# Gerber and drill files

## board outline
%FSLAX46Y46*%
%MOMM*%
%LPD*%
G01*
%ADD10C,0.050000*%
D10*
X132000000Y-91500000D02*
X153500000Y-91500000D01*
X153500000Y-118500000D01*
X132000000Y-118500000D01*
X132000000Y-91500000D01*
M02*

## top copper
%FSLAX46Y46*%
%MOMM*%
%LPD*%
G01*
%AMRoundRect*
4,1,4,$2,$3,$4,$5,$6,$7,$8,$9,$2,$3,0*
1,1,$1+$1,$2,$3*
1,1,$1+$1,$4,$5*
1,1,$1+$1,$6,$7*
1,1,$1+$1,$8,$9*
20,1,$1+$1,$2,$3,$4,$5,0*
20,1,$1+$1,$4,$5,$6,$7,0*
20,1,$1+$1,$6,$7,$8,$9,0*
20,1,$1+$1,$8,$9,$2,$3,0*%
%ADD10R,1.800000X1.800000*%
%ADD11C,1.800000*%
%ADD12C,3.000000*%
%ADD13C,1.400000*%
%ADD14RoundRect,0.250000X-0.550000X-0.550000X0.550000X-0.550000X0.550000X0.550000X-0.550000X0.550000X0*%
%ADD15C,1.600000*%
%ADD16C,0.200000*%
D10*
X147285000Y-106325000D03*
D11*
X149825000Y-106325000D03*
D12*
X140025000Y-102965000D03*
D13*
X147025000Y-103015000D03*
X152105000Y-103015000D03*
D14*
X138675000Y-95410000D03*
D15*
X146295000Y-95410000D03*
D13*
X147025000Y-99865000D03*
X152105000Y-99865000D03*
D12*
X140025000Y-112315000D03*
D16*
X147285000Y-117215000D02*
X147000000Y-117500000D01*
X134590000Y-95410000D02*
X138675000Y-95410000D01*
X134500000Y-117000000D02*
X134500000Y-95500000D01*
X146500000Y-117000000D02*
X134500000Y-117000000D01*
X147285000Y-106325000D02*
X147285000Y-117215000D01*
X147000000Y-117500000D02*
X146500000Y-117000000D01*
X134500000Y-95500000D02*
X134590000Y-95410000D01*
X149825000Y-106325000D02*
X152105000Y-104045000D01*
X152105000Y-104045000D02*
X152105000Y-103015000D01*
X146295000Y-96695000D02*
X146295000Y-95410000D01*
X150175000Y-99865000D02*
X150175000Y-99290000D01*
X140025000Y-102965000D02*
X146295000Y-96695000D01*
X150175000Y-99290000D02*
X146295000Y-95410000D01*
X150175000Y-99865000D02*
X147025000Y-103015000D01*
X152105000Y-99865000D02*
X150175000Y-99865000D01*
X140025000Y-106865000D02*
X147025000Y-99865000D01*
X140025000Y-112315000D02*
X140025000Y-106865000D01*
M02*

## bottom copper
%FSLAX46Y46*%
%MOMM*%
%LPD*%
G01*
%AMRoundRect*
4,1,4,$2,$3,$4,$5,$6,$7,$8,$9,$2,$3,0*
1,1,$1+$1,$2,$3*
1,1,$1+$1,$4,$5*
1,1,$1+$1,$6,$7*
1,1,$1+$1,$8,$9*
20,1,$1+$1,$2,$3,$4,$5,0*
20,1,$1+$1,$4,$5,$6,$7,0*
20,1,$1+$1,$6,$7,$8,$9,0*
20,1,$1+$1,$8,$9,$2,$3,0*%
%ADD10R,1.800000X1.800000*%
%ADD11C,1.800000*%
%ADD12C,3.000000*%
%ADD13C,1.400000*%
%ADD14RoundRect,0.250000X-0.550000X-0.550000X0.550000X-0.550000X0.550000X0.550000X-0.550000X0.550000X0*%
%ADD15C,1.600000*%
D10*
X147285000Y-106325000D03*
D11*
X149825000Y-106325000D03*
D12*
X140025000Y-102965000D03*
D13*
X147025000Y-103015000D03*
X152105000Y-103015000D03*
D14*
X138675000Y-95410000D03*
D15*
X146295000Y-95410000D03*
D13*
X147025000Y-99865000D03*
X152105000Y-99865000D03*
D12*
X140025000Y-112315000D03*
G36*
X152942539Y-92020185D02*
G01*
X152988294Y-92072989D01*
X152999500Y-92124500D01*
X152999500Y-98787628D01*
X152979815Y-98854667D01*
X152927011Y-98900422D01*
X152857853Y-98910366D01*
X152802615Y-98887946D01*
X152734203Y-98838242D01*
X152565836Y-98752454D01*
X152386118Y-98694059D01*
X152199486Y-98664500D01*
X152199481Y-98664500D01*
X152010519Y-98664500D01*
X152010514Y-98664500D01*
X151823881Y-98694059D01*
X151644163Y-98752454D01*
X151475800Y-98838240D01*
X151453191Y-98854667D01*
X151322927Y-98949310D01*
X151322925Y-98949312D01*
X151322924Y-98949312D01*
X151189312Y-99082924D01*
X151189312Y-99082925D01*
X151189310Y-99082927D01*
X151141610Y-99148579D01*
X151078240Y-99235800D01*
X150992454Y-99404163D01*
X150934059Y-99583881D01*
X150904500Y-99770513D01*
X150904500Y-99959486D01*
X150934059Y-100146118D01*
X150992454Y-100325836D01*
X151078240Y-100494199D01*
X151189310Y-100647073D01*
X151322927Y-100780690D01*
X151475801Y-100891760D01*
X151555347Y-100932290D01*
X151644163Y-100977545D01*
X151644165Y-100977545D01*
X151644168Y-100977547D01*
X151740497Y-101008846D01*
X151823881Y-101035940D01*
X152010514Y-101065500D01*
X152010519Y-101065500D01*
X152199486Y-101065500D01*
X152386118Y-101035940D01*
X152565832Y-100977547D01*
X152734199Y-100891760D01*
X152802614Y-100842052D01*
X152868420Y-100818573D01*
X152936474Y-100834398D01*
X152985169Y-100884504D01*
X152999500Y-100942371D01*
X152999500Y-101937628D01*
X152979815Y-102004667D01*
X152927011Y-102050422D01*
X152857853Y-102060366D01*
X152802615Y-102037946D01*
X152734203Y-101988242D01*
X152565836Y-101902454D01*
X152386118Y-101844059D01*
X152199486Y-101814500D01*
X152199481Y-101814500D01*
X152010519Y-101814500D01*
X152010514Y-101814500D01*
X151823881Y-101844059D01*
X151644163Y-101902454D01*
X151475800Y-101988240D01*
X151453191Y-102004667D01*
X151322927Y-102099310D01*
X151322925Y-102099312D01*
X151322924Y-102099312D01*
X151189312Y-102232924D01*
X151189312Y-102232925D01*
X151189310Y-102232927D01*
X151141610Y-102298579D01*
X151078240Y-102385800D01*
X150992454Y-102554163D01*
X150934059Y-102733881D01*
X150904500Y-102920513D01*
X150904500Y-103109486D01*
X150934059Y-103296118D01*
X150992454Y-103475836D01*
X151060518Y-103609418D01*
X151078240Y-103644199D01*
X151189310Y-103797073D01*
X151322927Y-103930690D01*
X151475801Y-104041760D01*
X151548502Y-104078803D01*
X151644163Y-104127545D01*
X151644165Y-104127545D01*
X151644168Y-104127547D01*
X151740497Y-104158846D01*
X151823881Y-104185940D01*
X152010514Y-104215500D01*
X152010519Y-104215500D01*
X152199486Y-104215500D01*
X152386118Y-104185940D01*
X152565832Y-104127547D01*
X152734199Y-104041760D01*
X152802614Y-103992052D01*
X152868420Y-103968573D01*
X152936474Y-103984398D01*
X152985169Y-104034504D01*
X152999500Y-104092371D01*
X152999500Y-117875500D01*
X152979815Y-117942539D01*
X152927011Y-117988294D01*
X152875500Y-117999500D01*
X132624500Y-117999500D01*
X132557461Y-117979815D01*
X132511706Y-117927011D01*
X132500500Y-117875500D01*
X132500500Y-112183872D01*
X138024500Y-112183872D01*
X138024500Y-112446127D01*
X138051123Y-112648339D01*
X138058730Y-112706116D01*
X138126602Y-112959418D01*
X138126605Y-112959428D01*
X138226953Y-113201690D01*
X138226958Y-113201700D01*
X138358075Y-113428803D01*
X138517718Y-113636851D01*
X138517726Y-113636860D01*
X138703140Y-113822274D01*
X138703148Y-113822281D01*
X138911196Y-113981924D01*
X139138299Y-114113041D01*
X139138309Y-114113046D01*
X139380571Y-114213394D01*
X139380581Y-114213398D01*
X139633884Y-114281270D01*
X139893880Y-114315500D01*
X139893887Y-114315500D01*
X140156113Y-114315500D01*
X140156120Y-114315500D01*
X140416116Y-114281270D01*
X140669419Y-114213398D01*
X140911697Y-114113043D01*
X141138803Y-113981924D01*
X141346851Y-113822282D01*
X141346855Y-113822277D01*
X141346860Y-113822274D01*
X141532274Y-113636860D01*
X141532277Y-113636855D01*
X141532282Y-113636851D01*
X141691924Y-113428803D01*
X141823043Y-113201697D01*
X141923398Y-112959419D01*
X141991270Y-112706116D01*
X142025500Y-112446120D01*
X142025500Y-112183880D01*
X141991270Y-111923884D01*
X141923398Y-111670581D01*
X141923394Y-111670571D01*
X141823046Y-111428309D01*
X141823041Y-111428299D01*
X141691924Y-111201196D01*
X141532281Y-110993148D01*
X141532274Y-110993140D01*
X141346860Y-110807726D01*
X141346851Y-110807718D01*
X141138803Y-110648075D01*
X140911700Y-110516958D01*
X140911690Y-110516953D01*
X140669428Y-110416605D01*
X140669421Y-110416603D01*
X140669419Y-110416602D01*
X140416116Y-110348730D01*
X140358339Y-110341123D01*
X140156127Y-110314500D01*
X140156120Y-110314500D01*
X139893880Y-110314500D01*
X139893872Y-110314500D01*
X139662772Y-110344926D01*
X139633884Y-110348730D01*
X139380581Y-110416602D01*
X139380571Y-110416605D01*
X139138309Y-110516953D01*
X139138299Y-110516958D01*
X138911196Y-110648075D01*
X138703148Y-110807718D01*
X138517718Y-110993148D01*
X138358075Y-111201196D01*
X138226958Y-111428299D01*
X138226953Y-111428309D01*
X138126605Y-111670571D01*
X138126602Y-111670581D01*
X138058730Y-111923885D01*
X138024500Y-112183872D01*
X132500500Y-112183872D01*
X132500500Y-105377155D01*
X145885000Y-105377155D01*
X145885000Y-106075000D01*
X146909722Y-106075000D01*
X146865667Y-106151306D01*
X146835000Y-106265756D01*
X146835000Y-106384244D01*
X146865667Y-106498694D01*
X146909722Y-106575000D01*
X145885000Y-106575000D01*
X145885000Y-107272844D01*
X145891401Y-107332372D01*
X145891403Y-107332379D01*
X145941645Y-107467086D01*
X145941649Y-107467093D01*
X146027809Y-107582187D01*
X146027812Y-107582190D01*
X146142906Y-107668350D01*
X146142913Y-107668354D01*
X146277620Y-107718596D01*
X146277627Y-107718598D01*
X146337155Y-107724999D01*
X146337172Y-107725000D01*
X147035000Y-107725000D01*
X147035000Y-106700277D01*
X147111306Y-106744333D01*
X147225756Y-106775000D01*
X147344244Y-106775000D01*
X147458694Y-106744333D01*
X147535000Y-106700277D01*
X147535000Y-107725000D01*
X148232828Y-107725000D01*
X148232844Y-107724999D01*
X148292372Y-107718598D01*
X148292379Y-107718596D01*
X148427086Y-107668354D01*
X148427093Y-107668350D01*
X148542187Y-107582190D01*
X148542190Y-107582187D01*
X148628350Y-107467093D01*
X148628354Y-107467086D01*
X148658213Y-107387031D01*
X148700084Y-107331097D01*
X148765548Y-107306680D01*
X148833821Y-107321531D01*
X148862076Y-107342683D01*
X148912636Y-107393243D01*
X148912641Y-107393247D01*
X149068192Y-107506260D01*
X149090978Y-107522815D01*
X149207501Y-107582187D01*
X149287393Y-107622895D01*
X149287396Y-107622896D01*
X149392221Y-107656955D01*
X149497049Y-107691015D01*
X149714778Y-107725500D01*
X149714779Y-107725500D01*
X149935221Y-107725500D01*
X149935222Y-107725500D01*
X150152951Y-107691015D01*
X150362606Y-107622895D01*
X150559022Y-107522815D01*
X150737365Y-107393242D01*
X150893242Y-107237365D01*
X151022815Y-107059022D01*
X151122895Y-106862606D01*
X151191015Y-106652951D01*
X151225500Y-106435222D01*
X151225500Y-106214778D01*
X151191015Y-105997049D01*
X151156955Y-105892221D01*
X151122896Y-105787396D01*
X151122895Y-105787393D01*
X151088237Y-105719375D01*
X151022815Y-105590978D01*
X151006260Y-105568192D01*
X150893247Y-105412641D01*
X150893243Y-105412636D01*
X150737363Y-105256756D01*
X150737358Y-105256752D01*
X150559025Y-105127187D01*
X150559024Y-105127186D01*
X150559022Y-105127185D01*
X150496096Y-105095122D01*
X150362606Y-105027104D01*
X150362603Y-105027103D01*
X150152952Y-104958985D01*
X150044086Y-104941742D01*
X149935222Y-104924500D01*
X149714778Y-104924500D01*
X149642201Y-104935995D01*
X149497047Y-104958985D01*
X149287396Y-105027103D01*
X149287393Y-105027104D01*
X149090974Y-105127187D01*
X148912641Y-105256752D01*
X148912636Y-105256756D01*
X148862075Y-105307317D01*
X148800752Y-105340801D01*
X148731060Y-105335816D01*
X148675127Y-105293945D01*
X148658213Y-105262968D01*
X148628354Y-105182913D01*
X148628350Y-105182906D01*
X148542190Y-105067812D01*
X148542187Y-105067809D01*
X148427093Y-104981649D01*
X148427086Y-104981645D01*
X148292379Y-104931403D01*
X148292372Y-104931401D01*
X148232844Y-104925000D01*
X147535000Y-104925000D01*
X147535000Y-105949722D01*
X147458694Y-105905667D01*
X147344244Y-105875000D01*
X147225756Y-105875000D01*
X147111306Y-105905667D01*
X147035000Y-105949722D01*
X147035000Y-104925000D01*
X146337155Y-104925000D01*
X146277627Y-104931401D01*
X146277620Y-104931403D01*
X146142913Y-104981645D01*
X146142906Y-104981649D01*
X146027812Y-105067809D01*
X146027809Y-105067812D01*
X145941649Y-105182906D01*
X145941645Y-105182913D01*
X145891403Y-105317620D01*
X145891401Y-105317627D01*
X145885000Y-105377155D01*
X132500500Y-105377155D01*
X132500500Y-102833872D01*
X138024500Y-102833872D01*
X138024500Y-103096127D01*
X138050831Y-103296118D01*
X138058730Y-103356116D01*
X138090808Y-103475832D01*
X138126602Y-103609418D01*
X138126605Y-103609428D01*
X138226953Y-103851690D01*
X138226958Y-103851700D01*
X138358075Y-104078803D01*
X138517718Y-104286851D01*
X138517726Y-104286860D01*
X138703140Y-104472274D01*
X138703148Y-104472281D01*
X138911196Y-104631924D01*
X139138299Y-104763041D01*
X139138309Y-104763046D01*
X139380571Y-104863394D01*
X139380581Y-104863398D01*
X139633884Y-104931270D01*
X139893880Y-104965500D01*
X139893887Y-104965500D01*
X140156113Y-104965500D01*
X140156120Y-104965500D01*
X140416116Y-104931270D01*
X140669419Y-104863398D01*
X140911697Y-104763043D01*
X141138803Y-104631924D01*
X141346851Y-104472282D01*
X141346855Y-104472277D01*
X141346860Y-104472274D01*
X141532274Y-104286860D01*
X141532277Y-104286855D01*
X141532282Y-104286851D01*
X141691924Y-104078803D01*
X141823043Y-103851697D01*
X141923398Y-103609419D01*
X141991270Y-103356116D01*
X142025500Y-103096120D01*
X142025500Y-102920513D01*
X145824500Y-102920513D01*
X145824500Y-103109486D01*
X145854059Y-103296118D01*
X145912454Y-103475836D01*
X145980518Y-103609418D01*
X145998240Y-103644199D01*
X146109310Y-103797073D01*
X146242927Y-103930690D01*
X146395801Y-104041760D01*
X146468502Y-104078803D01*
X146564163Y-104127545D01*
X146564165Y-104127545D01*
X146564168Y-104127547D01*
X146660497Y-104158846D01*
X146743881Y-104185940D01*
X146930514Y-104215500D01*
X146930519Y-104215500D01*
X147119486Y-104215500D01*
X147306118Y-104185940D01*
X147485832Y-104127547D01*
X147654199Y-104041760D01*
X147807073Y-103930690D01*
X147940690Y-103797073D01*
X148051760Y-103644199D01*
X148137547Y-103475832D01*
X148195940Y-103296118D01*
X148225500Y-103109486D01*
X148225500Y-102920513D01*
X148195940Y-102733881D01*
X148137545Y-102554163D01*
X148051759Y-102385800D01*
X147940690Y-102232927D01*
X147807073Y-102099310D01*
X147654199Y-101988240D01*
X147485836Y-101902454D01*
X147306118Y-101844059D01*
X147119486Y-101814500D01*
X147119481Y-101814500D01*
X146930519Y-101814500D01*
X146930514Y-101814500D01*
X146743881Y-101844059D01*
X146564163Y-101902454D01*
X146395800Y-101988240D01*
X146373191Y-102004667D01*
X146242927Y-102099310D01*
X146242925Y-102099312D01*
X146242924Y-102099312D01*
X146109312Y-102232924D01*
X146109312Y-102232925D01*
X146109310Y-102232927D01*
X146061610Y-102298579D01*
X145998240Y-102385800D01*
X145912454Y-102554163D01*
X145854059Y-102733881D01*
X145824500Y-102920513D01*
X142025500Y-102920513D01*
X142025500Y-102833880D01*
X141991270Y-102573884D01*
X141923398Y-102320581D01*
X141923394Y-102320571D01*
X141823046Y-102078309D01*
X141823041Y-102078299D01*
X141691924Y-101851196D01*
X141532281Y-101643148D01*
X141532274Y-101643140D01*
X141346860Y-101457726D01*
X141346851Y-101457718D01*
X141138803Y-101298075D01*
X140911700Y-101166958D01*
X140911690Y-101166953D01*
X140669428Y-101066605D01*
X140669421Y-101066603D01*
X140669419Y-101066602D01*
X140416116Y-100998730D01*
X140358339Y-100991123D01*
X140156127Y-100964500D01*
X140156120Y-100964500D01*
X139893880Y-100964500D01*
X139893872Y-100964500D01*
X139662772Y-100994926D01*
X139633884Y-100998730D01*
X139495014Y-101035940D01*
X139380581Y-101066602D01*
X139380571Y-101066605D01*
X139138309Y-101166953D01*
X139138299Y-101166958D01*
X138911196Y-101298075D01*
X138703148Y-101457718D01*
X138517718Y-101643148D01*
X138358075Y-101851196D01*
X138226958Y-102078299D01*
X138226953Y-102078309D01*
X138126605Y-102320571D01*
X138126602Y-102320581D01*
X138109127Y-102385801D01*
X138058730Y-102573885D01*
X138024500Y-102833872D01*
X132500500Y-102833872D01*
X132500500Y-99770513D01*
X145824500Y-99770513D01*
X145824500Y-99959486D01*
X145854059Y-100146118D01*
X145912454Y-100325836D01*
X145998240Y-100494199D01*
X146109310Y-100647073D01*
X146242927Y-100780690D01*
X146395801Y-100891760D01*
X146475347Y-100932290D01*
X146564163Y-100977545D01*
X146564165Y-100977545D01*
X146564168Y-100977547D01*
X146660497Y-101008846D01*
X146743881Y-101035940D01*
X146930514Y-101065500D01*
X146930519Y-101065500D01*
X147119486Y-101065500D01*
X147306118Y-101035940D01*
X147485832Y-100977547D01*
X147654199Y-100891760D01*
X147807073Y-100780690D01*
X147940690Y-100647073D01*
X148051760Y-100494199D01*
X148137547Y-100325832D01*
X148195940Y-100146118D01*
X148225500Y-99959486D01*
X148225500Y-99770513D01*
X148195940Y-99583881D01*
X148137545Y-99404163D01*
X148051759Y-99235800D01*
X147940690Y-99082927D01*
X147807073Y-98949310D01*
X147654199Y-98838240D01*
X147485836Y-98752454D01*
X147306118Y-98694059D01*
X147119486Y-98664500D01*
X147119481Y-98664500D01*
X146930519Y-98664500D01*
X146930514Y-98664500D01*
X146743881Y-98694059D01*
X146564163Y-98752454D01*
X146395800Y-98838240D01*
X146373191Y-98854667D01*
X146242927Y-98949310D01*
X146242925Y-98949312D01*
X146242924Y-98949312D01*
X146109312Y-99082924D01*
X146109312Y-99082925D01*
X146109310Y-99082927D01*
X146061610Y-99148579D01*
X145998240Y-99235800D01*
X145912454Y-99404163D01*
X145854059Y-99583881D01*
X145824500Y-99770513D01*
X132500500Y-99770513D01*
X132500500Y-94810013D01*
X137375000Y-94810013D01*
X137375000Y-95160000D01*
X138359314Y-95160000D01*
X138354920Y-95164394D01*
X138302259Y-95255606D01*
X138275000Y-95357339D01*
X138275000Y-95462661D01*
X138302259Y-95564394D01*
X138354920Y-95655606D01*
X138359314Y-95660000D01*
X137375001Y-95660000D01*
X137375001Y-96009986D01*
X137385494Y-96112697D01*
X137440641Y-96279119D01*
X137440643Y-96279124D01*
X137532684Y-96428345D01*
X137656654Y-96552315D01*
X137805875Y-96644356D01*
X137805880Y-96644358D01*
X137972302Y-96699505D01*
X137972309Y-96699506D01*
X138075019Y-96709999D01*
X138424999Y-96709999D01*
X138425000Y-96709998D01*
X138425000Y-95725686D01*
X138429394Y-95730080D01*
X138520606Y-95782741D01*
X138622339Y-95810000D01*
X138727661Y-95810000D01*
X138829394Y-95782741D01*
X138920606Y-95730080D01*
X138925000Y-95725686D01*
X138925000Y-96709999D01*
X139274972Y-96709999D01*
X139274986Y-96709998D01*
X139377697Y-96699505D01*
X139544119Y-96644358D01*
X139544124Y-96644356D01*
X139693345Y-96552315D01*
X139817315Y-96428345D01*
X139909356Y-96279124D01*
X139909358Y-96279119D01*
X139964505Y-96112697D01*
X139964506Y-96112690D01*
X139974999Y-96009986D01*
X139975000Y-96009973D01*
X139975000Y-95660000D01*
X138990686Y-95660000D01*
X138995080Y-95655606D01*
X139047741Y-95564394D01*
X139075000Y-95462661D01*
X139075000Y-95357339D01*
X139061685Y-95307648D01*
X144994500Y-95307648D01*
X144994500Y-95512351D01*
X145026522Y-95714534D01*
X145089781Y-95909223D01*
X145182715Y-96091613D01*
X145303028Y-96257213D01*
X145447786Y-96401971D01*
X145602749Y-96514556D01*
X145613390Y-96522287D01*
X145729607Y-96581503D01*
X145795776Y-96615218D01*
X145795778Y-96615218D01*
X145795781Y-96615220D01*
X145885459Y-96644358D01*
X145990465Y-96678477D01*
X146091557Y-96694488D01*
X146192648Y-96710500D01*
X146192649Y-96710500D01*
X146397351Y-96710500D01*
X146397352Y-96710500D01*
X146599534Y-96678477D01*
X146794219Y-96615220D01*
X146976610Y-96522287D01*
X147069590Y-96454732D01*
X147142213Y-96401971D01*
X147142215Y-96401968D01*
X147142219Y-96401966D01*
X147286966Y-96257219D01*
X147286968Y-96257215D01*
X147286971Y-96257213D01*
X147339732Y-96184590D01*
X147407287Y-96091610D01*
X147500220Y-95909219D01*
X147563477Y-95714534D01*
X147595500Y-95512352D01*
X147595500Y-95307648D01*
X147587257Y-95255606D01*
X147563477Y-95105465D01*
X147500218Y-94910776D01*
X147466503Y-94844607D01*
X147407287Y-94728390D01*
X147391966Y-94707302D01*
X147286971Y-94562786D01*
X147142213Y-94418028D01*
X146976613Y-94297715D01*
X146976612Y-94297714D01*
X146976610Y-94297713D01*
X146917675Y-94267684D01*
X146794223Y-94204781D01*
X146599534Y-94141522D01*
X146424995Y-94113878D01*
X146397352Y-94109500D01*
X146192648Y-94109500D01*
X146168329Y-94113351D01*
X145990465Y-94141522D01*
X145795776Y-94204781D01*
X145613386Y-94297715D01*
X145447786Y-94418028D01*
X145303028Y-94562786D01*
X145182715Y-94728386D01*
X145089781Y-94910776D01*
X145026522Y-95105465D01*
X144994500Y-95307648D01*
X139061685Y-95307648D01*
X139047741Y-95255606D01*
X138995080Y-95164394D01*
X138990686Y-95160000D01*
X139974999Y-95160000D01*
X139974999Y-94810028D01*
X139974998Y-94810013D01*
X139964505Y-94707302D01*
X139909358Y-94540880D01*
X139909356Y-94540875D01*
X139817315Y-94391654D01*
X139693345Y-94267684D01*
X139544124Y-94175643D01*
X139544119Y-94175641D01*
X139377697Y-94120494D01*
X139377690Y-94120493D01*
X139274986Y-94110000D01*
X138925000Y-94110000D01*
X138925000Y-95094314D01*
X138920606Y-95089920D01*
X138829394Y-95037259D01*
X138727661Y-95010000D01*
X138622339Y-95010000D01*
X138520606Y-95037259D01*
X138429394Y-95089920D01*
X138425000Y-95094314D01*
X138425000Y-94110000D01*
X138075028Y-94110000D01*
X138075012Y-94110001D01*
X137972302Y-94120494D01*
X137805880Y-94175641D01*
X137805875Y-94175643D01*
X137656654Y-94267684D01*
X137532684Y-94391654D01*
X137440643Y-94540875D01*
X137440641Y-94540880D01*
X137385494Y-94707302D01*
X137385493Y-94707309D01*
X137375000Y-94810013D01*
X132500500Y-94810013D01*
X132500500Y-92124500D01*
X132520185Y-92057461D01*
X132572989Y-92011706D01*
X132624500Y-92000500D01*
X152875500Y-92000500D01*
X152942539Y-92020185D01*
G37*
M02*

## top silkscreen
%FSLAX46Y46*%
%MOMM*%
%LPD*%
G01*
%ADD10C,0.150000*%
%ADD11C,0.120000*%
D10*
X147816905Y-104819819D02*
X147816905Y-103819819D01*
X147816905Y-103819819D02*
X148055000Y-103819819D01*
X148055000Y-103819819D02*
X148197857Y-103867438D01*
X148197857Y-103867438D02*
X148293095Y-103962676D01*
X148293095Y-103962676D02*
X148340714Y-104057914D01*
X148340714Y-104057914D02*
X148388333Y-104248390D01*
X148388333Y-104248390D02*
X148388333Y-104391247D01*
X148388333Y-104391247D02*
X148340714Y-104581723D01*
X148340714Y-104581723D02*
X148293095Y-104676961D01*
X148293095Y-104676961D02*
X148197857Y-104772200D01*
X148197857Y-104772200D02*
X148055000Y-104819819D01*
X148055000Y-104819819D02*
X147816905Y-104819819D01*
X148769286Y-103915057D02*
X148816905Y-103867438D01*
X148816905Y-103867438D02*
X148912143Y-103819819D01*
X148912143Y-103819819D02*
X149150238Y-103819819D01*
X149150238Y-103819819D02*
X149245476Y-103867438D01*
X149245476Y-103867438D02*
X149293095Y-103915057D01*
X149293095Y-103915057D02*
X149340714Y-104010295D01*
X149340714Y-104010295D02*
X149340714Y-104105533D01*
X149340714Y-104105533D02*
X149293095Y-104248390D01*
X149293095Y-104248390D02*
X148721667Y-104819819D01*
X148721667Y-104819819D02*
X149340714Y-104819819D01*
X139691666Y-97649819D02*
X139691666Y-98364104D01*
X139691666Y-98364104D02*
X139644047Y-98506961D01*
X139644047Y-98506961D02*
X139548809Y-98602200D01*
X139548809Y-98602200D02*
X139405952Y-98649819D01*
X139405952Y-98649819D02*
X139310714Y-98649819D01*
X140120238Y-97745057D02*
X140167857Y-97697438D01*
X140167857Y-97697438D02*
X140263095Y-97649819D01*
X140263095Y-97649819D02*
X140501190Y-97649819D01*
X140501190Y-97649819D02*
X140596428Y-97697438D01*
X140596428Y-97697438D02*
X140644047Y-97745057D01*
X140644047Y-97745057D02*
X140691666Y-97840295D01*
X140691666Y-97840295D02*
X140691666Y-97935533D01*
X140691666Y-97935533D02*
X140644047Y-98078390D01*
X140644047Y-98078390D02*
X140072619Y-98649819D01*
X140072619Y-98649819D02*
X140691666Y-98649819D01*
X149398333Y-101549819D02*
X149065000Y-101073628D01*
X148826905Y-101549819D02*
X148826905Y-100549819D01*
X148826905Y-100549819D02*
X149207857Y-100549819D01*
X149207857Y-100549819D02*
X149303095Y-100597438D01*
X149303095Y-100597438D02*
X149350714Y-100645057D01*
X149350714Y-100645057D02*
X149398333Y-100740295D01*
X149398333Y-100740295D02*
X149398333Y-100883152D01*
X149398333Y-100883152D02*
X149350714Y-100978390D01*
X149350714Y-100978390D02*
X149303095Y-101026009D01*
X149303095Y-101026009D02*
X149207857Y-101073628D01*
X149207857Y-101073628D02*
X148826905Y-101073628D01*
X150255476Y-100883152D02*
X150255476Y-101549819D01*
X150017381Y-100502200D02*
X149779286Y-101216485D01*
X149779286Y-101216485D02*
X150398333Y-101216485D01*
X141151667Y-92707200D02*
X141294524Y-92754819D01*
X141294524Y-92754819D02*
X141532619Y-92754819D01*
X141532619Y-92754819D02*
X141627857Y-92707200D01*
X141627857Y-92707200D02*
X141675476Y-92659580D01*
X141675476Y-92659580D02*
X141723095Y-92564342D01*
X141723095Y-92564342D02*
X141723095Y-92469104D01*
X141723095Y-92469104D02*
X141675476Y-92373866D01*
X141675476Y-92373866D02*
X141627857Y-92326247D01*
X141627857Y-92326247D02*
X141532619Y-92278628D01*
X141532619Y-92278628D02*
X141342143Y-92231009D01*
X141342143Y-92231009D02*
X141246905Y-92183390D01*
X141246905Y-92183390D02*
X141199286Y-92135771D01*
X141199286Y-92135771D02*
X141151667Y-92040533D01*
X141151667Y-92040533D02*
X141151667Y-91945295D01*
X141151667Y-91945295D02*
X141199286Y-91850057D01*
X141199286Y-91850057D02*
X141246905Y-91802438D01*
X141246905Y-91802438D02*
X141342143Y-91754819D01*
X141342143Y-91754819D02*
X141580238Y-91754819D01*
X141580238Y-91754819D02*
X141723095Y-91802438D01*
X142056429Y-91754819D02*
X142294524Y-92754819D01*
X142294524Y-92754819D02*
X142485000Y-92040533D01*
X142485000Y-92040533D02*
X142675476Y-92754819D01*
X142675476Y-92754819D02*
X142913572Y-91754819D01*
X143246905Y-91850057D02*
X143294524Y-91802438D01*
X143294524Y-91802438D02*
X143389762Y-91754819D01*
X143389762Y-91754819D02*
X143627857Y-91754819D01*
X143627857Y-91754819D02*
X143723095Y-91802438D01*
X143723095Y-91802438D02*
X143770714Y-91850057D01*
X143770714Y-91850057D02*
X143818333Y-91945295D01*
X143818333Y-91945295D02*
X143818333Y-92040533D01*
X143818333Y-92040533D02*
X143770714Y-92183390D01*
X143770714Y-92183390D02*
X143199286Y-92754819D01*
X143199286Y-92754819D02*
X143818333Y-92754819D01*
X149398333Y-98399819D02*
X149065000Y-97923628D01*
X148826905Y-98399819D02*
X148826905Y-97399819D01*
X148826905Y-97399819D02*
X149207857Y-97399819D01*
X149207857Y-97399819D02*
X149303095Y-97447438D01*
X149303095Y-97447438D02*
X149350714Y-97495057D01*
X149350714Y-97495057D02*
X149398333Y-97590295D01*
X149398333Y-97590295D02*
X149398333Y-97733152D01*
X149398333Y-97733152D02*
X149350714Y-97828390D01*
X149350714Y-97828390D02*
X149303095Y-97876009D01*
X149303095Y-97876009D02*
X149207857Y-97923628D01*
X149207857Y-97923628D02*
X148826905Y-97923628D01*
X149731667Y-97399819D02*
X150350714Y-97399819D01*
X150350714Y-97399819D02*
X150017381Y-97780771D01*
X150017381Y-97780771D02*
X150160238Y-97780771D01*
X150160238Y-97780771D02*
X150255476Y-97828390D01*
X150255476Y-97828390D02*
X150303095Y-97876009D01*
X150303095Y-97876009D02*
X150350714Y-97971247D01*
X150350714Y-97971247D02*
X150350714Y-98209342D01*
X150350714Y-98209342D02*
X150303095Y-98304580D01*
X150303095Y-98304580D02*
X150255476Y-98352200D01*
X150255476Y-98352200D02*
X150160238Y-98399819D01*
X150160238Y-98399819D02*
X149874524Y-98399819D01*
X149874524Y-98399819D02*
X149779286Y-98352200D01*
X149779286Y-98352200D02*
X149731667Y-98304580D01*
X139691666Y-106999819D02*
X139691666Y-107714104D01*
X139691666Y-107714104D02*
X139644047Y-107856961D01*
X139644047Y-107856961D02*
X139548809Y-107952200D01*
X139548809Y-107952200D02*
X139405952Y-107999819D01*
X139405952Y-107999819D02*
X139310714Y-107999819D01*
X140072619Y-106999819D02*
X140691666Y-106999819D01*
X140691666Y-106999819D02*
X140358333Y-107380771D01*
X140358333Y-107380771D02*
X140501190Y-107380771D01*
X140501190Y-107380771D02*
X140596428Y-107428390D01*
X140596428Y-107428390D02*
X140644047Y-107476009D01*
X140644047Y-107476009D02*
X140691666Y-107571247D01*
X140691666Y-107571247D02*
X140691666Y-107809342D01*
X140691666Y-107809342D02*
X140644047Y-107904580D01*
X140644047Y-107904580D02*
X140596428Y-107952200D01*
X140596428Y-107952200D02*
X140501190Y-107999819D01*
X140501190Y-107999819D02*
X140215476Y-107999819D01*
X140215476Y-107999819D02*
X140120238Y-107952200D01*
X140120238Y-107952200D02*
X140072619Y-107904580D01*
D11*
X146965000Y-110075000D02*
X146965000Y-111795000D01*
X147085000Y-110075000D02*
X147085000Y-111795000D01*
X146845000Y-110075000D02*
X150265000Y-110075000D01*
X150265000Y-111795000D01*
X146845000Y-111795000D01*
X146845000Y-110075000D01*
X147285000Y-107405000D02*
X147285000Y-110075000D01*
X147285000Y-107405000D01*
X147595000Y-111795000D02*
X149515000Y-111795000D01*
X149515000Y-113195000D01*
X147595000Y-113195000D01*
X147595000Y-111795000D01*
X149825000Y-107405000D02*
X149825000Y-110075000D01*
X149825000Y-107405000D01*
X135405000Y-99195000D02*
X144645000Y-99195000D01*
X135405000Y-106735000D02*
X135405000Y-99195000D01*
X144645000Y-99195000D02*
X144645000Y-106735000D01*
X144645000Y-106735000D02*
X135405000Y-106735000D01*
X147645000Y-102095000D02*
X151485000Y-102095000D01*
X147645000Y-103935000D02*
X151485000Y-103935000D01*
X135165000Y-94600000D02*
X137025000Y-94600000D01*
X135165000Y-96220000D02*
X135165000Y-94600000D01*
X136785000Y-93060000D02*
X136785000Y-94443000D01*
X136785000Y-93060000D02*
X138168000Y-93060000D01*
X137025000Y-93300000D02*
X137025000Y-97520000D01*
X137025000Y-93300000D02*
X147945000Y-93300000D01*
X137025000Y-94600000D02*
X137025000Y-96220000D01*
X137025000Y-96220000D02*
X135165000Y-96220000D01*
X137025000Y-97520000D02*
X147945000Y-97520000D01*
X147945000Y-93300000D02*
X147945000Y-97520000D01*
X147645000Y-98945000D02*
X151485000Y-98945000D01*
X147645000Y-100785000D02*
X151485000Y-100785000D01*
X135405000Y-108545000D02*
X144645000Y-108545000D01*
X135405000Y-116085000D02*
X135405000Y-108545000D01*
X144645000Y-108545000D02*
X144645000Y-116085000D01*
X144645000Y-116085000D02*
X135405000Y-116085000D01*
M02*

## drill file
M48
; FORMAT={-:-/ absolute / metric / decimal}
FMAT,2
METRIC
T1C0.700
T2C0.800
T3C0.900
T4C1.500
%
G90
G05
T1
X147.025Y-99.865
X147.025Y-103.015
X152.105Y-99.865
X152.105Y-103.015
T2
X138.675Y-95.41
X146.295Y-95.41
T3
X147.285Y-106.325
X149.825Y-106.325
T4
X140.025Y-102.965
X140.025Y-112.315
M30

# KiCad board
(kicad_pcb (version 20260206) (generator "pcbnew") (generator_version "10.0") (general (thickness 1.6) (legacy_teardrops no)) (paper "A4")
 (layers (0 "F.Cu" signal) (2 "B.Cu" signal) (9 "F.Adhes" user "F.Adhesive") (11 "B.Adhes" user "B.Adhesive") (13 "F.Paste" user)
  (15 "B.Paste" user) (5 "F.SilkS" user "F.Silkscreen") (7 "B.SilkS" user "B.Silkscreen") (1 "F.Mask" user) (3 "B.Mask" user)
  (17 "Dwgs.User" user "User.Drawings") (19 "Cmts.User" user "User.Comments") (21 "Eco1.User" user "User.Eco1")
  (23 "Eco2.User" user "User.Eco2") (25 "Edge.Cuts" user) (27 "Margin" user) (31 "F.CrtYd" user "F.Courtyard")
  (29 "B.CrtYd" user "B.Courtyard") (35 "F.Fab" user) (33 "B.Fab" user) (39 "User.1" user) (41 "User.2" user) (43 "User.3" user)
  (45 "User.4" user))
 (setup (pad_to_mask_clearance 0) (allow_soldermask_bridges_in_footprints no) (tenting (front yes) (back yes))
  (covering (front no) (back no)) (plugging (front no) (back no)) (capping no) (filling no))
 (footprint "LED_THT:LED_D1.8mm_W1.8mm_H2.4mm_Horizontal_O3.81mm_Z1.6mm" (layer "F.Cu") (at 147.285 106.325)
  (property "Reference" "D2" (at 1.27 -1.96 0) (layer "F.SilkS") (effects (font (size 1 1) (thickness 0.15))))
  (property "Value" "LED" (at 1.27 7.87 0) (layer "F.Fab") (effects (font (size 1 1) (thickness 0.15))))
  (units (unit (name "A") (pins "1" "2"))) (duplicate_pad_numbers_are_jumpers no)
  (fp_line (start -0.32 3.75) (end -0.32 5.47) (stroke (width 0.12) (type solid)) (layer "F.SilkS"))
  (fp_line (start -0.2 3.75) (end -0.2 5.47) (stroke (width 0.12) (type solid)) (layer "F.SilkS"))
  (fp_rect (start -0.44 3.75) (end 2.98 5.47) (stroke (width 0.12) (type solid)) (fill no) (layer "F.SilkS"))
  (fp_rect (start 0 1.08) (end 0 3.75) (stroke (width 0.12) (type solid)) (fill no) (layer "F.SilkS"))
  (fp_rect (start 0.31 5.47) (end 2.23 6.87) (stroke (width 0.12) (type solid)) (fill no) (layer "F.SilkS"))
  (fp_rect (start 2.54 1.08) (end 2.54 3.75) (stroke (width 0.12) (type solid)) (fill no) (layer "F.SilkS"))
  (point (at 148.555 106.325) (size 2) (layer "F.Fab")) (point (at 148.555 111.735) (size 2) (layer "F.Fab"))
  (pad "1" thru_hole rect (at 0 0) (size 1.8 1.8) (drill 0.9) (layers "*.Cu" "*.Mask") (remove_unused_layers no) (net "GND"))
  (pad "2" thru_hole circle (at 2.54 0) (size 1.8 1.8) (drill 0.9) (layers "*.Cu" "*.Mask") (remove_unused_layers no) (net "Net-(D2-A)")))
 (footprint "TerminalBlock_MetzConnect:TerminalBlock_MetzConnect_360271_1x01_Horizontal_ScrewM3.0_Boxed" (layer "F.Cu") (at 140.025 102.965)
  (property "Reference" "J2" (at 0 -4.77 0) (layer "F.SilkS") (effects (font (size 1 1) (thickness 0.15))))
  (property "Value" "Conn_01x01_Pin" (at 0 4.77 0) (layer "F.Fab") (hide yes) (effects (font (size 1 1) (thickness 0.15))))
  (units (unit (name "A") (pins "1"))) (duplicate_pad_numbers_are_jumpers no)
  (fp_line (start -4.62 -3.77) (end 4.62 -3.77) (stroke (width 0.12) (type solid)) (layer "F.SilkS"))
  (fp_line (start -4.62 3.77) (end -4.62 -3.77) (stroke (width 0.12) (type solid)) (layer "F.SilkS"))
  (fp_line (start 4.62 -3.77) (end 4.62 3.77) (stroke (width 0.12) (type solid)) (layer "F.SilkS"))
  (fp_line (start 4.62 3.77) (end -4.62 3.77) (stroke (width 0.12) (type solid)) (layer "F.SilkS"))
  (pad "1" thru_hole circle (at 0 0) (size 3 3) (drill 1.5) (layers "*.Cu" "*.Mask") (remove_unused_layers no) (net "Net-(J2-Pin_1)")))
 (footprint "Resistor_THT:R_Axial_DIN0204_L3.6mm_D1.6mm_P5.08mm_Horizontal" (layer "F.Cu") (at 147.025 103.015)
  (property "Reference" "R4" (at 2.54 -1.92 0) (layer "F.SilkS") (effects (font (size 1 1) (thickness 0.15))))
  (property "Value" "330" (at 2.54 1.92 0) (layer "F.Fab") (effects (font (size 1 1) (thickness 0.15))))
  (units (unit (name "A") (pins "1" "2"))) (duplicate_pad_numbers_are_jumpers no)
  (fp_line (start 0.62 -0.92) (end 4.46 -0.92) (stroke (width 0.12) (type solid)) (layer "F.SilkS"))
  (fp_line (start 0.62 0.92) (end 4.46 0.92) (stroke (width 0.12) (type solid)) (layer "F.SilkS"))
  (pad "1" thru_hole circle (at 0 0) (size 1.4 1.4) (drill 0.7) (layers "*.Cu" "*.Mask") (remove_unused_layers no) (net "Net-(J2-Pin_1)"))
  (pad "2" thru_hole circle (at 5.08 0) (size 1.4 1.4) (drill 0.7) (layers "*.Cu" "*.Mask") (remove_unused_layers no) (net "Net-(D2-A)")))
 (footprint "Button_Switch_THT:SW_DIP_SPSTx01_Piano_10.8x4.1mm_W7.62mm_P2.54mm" (layer "F.Cu") (at 138.675 95.41)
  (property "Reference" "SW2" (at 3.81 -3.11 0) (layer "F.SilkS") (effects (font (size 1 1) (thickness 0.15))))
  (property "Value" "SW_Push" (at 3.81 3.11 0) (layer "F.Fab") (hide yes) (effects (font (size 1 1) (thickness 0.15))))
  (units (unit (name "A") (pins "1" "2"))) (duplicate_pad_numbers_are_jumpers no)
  (fp_line (start -3.51 -0.81) (end -1.65 -0.81) (stroke (width 0.12) (type solid)) (layer "F.SilkS"))
  (fp_line (start -3.51 0.81) (end -3.51 -0.81) (stroke (width 0.12) (type solid)) (layer "F.SilkS"))
  (fp_line (start -1.89 -2.35) (end -1.89 -0.967) (stroke (width 0.12) (type solid)) (layer "F.SilkS"))
  (fp_line (start -1.89 -2.35) (end -0.507 -2.35) (stroke (width 0.12) (type solid)) (layer "F.SilkS"))
  (fp_line (start -1.65 -2.11) (end -1.65 2.11) (stroke (width 0.12) (type solid)) (layer "F.SilkS"))
  (fp_line (start -1.65 -2.11) (end 9.27 -2.11) (stroke (width 0.12) (type solid)) (layer "F.SilkS"))
  (fp_line (start -1.65 -0.81) (end -1.65 0.81) (stroke (width 0.12) (type solid)) (layer "F.SilkS"))
  (fp_line (start -1.65 0.81) (end -3.51 0.81) (stroke (width 0.12) (type solid)) (layer "F.SilkS"))
  (fp_line (start -1.65 2.11) (end 9.27 2.11) (stroke (width 0.12) (type solid)) (layer "F.SilkS"))
  (fp_line (start 9.27 -2.11) (end 9.27 2.11) (stroke (width 0.12) (type solid)) (layer "F.SilkS"))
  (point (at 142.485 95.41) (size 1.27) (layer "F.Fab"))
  (pad "1" thru_hole roundrect (at 0 0) (size 1.6 1.6) (drill 0.8) (layers "*.Cu" "*.Mask") (remove_unused_layers no)
   (roundrect_rratio 0.15625) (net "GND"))
  (pad "2" thru_hole circle (at 7.62 0) (size 1.6 1.6) (drill 0.8) (layers "*.Cu" "*.Mask") (remove_unused_layers no) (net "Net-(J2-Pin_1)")))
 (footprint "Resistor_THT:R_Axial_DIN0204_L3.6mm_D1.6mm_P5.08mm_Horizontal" (layer "F.Cu") (at 147.025 99.865)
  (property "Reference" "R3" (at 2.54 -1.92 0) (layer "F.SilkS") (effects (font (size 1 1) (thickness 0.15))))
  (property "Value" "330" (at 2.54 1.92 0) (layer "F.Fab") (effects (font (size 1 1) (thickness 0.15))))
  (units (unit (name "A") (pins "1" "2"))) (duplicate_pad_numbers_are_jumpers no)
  (fp_line (start 0.62 -0.92) (end 4.46 -0.92) (stroke (width 0.12) (type solid)) (layer "F.SilkS"))
  (fp_line (start 0.62 0.92) (end 4.46 0.92) (stroke (width 0.12) (type solid)) (layer "F.SilkS"))
  (pad "1" thru_hole circle (at 0 0) (size 1.4 1.4) (drill 0.7) (layers "*.Cu" "*.Mask") (remove_unused_layers no) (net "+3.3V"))
  (pad "2" thru_hole circle (at 5.08 0) (size 1.4 1.4) (drill 0.7) (layers "*.Cu" "*.Mask") (remove_unused_layers no) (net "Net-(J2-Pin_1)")))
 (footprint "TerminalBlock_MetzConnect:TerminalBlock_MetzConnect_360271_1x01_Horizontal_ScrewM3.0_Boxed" (layer "F.Cu") (at 140.025 112.315)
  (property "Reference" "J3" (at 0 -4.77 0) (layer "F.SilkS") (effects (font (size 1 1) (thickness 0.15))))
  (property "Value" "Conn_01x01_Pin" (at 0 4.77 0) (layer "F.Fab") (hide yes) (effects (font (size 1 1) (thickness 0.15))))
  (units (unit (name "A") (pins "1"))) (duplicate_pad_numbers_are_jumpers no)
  (fp_line (start -4.62 -3.77) (end 4.62 -3.77) (stroke (width 0.12) (type solid)) (layer "F.SilkS"))
  (fp_line (start -4.62 3.77) (end -4.62 -3.77) (stroke (width 0.12) (type solid)) (layer "F.SilkS"))
  (fp_line (start 4.62 -3.77) (end 4.62 3.77) (stroke (width 0.12) (type solid)) (layer "F.SilkS"))
  (fp_line (start 4.62 3.77) (end -4.62 3.77) (stroke (width 0.12) (type solid)) (layer "F.SilkS"))
  (pad "1" thru_hole circle (at 0 0) (size 3 3) (drill 1.5) (layers "*.Cu" "*.Mask") (remove_unused_layers no) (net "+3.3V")))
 (gr_rect (start 132 91.5) (end 153.5 118.5) (stroke (width 0.05) (type default)) (fill no) (layer "Edge.Cuts"))
 (segment (start 147.285 117.215) (end 147 117.5) (width 0.2) (layer "F.Cu") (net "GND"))
 (segment (start 134.59 95.41) (end 138.675 95.41) (width 0.2) (layer "F.Cu") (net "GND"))
 (segment (start 134.5 117) (end 134.5 95.5) (width 0.2) (layer "F.Cu") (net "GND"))
 (segment (start 146.5 117) (end 134.5 117) (width 0.2) (layer "F.Cu") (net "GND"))
 (segment (start 147.285 106.325) (end 147.285 117.215) (width 0.2) (layer "F.Cu") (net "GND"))
 (segment (start 147 117.5) (end 146.5 117) (width 0.2) (layer "F.Cu") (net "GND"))
 (segment (start 134.5 95.5) (end 134.59 95.41) (width 0.2) (layer "F.Cu") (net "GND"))
 (segment (start 149.825 106.325) (end 152.105 104.045) (width 0.2) (layer "F.Cu") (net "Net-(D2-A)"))
 (segment (start 152.105 104.045) (end 152.105 103.015) (width 0.2) (layer "F.Cu") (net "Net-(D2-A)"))
 (segment (start 146.295 96.695) (end 146.295 95.41) (width 0.2) (layer "F.Cu") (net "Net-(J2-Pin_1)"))
 (segment (start 150.175 99.865) (end 150.175 99.29) (width 0.2) (layer "F.Cu") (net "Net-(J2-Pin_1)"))
 (segment (start 140.025 102.965) (end 146.295 96.695) (width 0.2) (layer "F.Cu") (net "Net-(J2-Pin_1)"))
 (segment (start 150.175 99.29) (end 146.295 95.41) (width 0.2) (layer "F.Cu") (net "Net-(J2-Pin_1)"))
 (segment (start 150.175 99.865) (end 147.025 103.015) (width 0.2) (layer "F.Cu") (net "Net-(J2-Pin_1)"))
 (segment (start 152.105 99.865) (end 150.175 99.865) (width 0.2) (layer "F.Cu") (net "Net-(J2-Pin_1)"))
 (segment (start 140.025 106.865) (end 147.025 99.865) (width 0.2) (layer "F.Cu") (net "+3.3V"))
 (segment (start 140.025 112.315) (end 140.025 106.865) (width 0.2) (layer "F.Cu") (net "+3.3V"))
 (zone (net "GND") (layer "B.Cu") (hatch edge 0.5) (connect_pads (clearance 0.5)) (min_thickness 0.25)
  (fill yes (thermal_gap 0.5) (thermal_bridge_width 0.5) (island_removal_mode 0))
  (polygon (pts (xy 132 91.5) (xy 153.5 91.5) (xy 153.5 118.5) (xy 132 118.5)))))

